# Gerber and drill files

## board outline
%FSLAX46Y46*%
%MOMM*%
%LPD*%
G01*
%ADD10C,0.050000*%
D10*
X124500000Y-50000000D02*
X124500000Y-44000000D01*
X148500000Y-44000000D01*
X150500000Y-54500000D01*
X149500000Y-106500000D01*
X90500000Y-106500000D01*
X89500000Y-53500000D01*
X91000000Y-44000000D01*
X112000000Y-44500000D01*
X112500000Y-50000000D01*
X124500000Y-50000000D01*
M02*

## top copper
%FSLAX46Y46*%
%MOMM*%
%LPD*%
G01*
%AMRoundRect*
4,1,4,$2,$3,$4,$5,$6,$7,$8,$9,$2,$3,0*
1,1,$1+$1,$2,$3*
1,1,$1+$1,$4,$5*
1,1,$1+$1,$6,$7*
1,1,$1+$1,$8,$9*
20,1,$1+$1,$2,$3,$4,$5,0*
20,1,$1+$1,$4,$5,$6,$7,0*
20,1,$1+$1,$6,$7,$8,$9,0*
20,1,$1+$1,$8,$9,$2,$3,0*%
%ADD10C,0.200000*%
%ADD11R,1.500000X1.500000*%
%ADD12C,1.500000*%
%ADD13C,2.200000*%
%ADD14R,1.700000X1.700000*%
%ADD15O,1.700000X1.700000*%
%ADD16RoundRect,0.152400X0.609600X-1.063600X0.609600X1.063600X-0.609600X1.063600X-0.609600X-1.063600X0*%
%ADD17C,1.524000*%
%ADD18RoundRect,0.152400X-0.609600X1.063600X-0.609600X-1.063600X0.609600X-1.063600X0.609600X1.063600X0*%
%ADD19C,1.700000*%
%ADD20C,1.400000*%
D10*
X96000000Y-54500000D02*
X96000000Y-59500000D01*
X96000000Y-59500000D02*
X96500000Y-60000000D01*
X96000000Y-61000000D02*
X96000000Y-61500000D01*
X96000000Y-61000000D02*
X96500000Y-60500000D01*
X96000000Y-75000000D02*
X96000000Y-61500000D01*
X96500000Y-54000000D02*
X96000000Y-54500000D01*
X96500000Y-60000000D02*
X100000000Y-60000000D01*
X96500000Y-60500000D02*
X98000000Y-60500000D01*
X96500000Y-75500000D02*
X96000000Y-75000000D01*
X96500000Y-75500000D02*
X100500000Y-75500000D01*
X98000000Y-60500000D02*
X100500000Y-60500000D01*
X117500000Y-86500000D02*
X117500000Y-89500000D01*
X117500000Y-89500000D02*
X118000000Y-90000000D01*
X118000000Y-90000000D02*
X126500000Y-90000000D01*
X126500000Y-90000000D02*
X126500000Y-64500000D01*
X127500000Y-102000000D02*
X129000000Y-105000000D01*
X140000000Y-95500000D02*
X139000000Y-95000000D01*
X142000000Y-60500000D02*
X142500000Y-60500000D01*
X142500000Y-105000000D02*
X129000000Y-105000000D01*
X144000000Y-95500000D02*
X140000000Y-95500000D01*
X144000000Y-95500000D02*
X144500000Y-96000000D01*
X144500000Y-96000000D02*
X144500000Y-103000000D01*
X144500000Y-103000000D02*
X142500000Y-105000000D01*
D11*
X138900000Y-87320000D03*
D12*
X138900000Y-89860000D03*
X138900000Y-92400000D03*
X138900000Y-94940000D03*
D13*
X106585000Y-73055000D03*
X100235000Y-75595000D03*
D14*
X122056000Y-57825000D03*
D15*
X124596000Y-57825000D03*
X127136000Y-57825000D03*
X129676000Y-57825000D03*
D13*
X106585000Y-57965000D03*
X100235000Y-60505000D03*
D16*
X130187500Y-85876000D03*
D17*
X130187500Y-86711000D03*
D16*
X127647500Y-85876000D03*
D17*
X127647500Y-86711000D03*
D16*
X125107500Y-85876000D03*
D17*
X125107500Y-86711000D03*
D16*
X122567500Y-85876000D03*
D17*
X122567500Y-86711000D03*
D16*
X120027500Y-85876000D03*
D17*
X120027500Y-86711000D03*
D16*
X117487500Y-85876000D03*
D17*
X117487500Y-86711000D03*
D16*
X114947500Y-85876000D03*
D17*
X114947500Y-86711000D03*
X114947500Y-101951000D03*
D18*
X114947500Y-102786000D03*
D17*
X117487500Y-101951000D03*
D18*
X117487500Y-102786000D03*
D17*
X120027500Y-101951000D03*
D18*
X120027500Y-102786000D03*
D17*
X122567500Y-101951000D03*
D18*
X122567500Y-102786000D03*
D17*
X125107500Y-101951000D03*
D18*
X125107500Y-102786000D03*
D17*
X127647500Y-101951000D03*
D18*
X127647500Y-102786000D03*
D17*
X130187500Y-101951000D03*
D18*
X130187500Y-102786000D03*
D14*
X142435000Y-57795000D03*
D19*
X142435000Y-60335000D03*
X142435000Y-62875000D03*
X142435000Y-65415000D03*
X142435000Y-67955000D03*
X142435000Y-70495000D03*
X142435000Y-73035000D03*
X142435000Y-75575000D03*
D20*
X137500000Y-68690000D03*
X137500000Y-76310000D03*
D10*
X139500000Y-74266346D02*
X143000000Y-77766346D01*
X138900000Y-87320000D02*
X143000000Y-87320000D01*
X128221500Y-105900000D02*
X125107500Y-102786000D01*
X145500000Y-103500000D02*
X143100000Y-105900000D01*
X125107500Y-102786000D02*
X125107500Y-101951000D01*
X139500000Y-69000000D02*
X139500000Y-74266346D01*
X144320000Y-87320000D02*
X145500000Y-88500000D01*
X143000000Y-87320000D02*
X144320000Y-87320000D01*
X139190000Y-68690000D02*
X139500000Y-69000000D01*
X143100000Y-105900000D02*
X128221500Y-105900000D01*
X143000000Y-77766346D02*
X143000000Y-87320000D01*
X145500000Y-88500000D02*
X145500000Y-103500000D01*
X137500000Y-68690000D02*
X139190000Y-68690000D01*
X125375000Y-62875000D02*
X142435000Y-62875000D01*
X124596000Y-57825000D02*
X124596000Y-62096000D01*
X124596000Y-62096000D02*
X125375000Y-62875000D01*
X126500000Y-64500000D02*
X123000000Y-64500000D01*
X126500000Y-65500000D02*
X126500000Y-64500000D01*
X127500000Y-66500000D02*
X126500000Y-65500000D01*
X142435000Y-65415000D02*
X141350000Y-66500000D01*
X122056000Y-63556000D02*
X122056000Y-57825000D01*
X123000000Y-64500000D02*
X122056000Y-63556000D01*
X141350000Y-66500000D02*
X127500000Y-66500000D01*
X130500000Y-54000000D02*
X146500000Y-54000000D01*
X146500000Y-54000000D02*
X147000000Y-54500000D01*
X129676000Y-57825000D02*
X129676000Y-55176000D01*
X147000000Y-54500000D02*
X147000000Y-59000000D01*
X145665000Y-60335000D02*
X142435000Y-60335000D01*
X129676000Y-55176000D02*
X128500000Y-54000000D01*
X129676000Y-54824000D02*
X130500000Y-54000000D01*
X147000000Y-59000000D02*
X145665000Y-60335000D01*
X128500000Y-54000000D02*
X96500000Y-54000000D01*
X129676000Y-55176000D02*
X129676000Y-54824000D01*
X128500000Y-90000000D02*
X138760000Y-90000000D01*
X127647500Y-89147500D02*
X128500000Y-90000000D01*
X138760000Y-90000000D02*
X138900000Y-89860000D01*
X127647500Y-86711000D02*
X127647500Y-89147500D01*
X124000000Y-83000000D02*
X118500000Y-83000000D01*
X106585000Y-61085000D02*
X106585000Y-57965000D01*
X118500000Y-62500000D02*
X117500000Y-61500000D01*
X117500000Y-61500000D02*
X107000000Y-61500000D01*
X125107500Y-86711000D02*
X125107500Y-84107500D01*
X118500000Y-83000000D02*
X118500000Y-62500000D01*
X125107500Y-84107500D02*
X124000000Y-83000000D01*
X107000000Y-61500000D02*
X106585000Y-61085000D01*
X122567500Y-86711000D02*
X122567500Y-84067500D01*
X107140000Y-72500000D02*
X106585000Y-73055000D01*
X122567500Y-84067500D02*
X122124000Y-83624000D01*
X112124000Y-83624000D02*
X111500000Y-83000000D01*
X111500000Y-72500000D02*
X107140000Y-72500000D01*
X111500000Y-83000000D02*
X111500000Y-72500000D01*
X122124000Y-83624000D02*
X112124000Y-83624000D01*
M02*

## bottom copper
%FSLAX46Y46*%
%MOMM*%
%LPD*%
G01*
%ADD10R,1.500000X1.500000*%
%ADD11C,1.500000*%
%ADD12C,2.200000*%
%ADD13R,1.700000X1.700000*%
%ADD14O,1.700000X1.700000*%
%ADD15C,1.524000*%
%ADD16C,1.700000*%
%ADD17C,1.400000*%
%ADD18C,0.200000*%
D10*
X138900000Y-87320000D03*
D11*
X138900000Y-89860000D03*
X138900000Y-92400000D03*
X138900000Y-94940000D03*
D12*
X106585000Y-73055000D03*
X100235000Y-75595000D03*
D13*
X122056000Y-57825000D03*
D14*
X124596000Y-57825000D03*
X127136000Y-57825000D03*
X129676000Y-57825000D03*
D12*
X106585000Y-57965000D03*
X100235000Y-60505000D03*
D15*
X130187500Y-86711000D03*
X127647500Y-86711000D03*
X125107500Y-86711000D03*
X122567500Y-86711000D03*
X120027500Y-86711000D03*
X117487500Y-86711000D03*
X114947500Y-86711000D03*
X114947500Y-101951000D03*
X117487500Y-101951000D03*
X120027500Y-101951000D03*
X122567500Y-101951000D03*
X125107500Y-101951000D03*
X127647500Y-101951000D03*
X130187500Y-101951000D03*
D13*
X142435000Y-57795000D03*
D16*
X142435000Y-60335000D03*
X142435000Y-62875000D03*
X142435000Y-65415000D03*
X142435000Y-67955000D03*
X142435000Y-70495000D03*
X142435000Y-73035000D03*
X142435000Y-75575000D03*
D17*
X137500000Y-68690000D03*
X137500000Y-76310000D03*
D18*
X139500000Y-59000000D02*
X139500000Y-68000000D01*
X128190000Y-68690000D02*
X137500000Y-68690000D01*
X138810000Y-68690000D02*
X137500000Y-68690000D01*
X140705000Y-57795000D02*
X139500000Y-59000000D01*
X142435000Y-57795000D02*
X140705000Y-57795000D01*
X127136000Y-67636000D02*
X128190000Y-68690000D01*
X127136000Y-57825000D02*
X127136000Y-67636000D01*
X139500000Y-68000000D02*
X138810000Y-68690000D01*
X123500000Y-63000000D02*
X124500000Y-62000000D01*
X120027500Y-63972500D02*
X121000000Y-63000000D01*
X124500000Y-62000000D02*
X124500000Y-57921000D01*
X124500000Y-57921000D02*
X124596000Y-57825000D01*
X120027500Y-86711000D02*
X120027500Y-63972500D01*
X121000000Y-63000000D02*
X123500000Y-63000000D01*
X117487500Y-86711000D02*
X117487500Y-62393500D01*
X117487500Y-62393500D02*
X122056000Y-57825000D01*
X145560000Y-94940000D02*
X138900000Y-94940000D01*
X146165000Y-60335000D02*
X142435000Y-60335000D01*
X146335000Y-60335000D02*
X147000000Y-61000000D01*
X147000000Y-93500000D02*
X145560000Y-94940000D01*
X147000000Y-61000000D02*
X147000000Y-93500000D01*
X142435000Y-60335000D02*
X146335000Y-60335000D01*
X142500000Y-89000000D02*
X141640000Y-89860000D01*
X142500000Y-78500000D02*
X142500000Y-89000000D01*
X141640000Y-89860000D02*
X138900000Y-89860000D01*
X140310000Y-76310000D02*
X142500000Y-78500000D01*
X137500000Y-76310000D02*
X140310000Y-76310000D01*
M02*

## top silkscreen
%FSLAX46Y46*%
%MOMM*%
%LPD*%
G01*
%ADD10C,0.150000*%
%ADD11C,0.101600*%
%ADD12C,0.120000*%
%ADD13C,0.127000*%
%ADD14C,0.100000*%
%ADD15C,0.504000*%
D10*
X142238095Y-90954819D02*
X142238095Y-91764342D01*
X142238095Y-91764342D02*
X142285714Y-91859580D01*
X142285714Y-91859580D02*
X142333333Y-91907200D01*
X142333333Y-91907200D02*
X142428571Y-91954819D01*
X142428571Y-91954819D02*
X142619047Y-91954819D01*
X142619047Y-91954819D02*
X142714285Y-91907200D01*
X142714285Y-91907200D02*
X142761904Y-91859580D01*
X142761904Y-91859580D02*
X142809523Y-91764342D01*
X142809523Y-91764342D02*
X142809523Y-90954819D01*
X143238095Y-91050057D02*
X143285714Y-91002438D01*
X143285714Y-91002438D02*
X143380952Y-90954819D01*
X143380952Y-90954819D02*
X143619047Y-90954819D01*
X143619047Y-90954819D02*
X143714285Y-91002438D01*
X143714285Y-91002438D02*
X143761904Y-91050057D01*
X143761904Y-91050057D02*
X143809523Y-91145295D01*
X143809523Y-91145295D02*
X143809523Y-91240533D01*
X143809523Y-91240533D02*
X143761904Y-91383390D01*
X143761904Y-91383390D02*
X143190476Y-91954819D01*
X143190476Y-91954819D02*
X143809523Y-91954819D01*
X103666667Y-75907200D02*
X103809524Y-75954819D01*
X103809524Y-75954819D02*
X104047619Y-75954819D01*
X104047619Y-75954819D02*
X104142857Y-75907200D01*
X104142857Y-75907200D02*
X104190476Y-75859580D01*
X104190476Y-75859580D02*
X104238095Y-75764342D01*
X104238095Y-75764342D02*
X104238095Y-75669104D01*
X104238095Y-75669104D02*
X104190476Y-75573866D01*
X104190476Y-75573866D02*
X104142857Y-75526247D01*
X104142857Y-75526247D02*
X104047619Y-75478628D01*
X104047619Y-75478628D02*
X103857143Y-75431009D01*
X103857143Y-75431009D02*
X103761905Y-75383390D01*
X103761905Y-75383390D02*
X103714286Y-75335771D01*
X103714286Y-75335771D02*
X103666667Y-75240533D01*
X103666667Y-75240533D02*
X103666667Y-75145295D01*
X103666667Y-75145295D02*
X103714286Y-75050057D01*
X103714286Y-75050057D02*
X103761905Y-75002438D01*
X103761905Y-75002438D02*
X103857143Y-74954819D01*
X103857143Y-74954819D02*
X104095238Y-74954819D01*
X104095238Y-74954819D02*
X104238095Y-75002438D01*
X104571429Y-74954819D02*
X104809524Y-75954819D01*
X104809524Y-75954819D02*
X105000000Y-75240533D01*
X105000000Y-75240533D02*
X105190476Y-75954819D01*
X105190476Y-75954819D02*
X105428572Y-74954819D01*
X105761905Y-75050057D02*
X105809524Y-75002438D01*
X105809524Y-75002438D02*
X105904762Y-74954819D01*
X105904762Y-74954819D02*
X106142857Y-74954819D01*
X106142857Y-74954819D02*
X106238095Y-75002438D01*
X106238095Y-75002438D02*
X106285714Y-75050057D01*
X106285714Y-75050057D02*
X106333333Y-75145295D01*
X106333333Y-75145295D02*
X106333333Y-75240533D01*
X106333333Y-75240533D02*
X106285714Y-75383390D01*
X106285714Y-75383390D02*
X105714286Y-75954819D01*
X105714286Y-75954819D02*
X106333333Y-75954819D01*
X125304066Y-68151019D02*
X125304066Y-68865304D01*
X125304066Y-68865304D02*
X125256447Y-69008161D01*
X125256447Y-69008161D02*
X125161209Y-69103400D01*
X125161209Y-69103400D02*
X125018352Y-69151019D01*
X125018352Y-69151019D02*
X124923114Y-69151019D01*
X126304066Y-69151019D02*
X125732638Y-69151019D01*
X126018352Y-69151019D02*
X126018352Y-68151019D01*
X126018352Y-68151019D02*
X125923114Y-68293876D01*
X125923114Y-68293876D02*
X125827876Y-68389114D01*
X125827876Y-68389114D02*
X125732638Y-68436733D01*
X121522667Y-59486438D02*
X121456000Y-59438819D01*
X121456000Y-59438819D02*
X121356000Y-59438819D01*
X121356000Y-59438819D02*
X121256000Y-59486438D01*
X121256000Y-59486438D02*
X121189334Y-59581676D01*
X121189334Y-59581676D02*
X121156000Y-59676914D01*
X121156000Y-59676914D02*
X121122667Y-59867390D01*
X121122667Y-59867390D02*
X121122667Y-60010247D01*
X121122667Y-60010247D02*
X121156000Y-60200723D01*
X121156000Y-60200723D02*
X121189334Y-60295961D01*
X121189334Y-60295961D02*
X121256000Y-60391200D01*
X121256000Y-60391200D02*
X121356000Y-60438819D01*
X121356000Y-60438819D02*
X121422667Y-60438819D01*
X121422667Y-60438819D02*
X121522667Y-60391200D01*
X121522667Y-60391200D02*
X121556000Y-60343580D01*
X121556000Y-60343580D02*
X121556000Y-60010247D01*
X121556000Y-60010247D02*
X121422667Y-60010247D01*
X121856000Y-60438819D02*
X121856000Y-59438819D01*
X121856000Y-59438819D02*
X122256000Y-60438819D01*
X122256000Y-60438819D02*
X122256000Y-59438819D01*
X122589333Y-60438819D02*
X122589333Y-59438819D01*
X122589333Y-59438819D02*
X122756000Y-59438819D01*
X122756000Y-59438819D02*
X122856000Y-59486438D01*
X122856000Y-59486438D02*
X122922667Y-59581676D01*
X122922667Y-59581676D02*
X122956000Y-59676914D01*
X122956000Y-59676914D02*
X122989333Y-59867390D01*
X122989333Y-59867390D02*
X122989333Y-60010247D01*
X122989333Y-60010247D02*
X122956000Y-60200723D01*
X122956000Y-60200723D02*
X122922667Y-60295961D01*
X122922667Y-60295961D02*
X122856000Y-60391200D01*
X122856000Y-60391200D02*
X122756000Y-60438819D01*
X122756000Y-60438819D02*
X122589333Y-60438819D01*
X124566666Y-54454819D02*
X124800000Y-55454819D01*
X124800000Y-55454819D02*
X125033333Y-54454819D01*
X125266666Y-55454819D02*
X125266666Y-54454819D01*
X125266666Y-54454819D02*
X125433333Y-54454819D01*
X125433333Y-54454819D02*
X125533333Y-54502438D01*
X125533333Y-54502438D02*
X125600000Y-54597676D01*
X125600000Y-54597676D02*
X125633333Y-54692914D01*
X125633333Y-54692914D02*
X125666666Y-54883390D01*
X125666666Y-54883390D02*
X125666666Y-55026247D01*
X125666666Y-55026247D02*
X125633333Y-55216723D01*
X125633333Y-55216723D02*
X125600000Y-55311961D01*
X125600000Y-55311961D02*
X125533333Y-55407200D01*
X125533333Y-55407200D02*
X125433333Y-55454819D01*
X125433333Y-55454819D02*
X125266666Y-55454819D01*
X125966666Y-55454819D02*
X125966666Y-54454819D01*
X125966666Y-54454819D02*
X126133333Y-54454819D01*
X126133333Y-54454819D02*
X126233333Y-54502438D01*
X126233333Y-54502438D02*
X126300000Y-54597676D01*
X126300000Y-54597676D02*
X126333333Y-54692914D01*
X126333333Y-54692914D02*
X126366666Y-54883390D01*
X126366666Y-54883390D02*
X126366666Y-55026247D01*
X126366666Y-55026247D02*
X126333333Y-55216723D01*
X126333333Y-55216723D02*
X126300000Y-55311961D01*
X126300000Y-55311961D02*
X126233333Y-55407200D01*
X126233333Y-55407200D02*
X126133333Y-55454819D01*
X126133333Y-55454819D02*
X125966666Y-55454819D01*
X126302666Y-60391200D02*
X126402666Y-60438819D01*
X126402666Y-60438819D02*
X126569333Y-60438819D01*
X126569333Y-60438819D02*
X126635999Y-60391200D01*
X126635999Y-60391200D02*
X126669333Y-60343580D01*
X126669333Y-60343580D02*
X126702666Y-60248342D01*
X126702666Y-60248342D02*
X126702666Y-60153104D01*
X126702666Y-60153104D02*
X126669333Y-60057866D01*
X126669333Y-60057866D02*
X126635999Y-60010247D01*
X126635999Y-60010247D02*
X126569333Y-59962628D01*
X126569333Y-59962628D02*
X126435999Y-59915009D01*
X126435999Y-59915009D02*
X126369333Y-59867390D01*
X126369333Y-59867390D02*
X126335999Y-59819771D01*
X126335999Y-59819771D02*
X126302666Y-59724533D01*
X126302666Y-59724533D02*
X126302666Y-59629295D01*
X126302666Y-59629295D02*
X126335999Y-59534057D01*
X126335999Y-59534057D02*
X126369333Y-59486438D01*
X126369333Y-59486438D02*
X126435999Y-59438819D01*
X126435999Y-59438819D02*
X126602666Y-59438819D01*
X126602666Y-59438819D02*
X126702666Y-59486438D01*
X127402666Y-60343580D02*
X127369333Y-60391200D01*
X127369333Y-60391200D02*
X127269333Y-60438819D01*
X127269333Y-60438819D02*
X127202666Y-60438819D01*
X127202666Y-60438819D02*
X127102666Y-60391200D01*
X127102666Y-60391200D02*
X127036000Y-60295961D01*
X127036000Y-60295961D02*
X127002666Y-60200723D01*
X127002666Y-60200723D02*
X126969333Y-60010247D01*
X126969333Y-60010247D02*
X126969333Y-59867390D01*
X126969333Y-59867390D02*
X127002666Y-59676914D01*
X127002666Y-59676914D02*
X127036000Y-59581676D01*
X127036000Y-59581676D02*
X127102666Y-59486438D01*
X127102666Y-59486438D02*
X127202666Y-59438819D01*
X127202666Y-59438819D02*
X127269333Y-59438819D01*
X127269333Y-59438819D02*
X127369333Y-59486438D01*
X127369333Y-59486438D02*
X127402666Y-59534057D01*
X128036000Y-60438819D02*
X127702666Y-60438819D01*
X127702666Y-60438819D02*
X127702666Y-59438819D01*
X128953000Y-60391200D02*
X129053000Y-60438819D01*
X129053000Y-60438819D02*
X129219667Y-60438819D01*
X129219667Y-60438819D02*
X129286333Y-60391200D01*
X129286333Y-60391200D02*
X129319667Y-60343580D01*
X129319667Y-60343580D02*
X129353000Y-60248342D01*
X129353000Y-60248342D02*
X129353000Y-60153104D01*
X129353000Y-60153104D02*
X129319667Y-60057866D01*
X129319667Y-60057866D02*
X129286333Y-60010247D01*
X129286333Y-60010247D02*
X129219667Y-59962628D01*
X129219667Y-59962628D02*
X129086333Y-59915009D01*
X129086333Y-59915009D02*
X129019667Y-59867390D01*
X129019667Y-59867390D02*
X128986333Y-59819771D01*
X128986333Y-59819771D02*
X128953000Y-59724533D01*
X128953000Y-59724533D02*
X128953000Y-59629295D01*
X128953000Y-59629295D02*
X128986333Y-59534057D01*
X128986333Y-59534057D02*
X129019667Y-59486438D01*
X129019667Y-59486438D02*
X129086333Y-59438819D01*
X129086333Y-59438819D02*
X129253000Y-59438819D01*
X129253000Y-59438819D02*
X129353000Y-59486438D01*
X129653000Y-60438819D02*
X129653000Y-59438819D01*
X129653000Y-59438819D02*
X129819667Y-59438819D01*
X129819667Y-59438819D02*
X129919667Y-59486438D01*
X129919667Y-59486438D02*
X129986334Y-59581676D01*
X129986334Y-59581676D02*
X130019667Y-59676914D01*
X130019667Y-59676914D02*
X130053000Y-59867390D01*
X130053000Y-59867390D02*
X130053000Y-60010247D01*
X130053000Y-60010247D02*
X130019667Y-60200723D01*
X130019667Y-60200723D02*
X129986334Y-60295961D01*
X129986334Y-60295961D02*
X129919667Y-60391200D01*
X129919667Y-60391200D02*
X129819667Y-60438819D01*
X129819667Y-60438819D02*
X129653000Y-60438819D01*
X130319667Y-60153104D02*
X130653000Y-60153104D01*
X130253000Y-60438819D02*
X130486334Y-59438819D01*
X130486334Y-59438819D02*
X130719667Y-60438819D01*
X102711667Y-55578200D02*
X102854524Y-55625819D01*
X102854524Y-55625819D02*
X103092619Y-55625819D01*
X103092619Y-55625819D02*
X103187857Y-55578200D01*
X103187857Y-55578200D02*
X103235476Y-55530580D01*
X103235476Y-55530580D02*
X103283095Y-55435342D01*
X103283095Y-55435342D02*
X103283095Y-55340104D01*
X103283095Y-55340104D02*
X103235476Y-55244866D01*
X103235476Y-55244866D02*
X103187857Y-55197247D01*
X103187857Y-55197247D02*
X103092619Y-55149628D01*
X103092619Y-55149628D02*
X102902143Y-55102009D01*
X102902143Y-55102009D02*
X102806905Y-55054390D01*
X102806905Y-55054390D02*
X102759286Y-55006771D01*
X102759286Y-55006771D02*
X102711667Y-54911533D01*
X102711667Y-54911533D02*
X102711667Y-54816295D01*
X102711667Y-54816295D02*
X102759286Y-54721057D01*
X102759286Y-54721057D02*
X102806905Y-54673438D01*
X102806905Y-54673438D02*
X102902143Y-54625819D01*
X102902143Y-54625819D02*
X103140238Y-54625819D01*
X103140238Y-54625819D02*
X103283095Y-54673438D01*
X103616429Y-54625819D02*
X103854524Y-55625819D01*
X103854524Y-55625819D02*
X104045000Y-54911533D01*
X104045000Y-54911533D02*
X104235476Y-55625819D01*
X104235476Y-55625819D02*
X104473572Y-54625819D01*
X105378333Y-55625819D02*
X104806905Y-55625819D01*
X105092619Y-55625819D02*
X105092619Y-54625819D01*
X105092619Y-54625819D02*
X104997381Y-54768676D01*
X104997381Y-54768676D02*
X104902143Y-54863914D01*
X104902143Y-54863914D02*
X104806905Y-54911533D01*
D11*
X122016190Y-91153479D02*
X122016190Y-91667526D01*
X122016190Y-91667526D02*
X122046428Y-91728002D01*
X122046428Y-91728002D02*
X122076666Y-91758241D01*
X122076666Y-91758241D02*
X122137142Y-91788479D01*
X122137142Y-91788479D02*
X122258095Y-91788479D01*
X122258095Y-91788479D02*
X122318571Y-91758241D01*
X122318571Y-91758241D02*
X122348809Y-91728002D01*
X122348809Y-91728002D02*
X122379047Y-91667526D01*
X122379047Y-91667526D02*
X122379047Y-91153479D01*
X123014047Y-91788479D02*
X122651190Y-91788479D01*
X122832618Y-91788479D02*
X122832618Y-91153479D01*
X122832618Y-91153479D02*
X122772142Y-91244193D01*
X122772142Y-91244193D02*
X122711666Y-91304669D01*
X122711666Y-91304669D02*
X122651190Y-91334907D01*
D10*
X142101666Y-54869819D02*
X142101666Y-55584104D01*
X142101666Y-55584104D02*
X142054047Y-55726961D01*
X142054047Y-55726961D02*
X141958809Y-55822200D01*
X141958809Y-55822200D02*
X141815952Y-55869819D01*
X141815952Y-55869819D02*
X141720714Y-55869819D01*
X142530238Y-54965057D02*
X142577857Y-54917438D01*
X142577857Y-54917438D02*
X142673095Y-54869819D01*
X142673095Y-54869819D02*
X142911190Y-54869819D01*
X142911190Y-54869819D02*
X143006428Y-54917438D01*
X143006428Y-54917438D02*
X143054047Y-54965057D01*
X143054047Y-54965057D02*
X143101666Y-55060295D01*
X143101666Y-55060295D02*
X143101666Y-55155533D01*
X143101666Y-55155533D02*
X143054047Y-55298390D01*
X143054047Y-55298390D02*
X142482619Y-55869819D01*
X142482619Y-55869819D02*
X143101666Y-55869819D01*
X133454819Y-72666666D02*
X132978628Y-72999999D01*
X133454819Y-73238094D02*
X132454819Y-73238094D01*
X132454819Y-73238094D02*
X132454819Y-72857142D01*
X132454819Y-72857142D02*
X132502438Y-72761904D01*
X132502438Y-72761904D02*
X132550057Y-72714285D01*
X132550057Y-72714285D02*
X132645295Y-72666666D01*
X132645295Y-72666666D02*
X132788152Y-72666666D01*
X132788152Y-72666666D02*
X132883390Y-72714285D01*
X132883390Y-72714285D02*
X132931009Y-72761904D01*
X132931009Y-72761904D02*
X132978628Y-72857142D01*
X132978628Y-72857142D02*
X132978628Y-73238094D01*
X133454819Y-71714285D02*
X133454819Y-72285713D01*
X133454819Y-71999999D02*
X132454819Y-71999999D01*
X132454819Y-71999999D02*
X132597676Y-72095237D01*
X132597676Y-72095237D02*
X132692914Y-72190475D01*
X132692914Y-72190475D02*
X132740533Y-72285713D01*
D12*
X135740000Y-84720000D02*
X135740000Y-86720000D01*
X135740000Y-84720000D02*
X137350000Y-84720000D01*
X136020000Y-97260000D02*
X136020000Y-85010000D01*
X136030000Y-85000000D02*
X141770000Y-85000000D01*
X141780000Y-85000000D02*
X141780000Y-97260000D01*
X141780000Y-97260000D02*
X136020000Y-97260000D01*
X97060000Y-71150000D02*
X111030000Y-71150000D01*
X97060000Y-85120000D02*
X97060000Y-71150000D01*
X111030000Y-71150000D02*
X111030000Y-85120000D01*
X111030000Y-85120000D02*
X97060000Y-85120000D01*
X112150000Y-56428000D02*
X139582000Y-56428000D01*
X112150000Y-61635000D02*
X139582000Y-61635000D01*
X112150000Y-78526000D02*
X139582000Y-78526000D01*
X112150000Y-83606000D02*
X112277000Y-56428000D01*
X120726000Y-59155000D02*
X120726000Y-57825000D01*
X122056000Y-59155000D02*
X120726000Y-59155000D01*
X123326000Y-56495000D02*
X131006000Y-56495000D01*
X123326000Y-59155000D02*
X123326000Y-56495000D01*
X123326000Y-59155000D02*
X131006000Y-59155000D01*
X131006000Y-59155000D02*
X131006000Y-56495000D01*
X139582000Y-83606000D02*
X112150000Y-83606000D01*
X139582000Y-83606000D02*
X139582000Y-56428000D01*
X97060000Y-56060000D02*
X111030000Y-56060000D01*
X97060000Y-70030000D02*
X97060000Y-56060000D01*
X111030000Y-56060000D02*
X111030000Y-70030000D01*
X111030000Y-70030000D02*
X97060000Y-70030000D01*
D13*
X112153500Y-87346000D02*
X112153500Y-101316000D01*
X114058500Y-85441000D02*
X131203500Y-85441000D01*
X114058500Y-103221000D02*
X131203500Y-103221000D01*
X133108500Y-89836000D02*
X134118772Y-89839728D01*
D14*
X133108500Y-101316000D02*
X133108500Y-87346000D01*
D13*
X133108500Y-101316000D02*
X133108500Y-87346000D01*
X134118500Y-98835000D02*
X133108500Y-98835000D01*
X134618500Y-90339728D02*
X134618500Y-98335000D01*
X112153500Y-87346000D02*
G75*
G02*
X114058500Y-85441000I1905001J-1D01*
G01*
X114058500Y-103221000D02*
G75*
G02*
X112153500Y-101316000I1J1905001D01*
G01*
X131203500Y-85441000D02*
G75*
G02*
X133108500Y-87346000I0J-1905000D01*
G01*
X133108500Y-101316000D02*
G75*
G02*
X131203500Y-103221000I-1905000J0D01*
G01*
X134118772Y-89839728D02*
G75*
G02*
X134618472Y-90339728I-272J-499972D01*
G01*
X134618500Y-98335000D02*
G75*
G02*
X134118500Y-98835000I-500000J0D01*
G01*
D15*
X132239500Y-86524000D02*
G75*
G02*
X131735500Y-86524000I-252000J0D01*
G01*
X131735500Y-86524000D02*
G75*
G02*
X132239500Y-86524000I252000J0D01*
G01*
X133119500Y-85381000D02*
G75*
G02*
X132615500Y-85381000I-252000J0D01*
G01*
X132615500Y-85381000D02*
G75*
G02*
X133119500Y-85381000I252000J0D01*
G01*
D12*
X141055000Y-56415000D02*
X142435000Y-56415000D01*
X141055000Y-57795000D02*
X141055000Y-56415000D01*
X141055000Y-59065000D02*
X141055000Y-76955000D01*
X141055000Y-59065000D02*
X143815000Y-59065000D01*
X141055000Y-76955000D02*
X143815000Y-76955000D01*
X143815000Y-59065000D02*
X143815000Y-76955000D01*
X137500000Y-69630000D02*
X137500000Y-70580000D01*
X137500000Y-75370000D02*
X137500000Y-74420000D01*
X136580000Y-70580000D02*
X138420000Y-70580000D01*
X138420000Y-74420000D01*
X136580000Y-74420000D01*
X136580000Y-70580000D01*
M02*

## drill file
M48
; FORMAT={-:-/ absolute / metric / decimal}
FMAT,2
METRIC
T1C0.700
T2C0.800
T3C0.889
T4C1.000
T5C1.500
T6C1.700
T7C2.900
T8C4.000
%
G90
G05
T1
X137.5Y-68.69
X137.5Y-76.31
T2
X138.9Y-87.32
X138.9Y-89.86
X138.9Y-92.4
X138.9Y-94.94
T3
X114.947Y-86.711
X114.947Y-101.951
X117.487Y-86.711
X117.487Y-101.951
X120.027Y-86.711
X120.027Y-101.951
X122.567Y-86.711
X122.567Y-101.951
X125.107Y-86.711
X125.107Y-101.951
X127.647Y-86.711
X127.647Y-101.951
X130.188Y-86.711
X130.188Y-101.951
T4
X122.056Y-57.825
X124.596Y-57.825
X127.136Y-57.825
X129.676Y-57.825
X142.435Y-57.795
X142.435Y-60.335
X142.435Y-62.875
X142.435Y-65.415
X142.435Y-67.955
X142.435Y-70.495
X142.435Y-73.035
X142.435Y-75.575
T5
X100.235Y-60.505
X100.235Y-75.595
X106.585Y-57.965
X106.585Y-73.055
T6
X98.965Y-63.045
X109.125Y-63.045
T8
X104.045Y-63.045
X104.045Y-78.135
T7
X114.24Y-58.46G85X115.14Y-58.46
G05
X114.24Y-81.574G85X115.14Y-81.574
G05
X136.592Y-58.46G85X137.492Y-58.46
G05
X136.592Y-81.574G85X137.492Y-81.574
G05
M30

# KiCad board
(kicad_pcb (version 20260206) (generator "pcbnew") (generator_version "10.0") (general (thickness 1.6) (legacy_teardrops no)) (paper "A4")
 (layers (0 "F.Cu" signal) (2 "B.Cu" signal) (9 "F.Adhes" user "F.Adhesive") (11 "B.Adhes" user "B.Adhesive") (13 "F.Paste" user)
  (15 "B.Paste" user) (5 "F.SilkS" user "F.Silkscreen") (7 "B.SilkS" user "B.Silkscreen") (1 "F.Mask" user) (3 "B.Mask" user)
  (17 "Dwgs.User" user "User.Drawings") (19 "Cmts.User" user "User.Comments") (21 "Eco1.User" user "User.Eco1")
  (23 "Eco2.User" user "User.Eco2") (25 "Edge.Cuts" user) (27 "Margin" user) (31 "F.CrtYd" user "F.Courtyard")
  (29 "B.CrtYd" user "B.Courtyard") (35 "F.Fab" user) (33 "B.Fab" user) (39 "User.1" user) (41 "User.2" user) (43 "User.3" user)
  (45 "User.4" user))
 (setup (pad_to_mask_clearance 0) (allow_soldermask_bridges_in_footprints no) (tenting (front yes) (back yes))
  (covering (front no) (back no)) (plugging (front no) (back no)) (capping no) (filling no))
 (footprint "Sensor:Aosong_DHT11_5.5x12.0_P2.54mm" (layer "F.Cu") (at 138.9 87.32)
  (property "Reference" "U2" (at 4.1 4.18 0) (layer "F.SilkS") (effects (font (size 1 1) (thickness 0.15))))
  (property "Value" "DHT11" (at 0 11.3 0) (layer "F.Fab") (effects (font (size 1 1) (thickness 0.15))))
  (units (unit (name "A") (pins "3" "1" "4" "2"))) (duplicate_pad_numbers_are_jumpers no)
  (fp_line (start -3.16 -2.6) (end -3.16 -0.6) (stroke (width 0.12) (type solid)) (layer "F.SilkS"))
  (fp_line (start -3.16 -2.6) (end -1.55 -2.6) (stroke (width 0.12) (type solid)) (layer "F.SilkS"))
  (fp_line (start -2.88 9.94) (end -2.88 -2.31) (stroke (width 0.12) (type solid)) (layer "F.SilkS"))
  (fp_line (start -2.87 -2.32) (end 2.87 -2.32) (stroke (width 0.12) (type solid)) (layer "F.SilkS"))
  (fp_line (start 2.88 -2.32) (end 2.88 9.94) (stroke (width 0.12) (type solid)) (layer "F.SilkS"))
  (fp_line (start 2.88 9.94) (end -2.88 9.94) (stroke (width 0.12) (type solid)) (layer "F.SilkS"))
  (pad "1" thru_hole rect (at 0 0) (size 1.5 1.5) (drill 0.8) (layers "*.Cu" "*.Mask") (remove_unused_layers no) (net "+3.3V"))
  (pad "2" thru_hole circle (at 0 2.54) (size 1.5 1.5) (drill 0.8) (layers "*.Cu" "*.Mask") (remove_unused_layers no) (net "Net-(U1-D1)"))
  (pad "3" thru_hole circle (at 0 5.08) (size 1.5 1.5) (drill 0.8) (layers "*.Cu" "*.Mask") (remove_unused_layers no)
   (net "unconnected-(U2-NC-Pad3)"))
  (pad "4" thru_hole circle (at 0 7.62) (size 1.5 1.5) (drill 0.8) (layers "*.Cu" "*.Mask") (remove_unused_layers no) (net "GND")))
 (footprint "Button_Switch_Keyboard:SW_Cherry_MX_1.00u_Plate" (layer "F.Cu") (at 106.585 73.055)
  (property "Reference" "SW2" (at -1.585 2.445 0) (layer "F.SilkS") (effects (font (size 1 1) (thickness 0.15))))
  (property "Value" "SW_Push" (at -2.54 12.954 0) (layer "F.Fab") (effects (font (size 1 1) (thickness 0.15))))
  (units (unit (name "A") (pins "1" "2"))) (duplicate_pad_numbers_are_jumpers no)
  (fp_line (start -9.525 -1.905) (end 4.445 -1.905) (stroke (width 0.12) (type solid)) (layer "F.SilkS"))
  (fp_line (start -9.525 12.065) (end -9.525 -1.905) (stroke (width 0.12) (type solid)) (layer "F.SilkS"))
  (fp_line (start 4.445 -1.905) (end 4.445 12.065) (stroke (width 0.12) (type solid)) (layer "F.SilkS"))
  (fp_line (start 4.445 12.065) (end -9.525 12.065) (stroke (width 0.12) (type solid)) (layer "F.SilkS"))
  (pad "" np_thru_hole circle (at -2.54 5.08) (size 4 4) (drill 4) (layers "*.Cu" "*.Mask"))
  (pad "1" thru_hole circle (at 0 0) (size 2.2 2.2) (drill 1.5) (layers "*.Cu" "*.Mask") (remove_unused_layers no) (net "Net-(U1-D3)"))
  (pad "2" thru_hole circle (at -6.35 2.54) (size 2.2 2.2) (drill 1.5) (layers "*.Cu" "*.Mask") (remove_unused_layers no) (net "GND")))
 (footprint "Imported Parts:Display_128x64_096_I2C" (layer "F.Cu") (at 125.866 57.825)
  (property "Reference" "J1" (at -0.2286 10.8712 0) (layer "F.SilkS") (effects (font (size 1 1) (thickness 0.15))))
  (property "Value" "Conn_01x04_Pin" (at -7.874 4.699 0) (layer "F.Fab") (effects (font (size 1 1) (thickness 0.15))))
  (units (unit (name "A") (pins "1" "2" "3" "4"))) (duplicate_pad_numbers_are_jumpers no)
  (fp_line (start -13.716 -1.397) (end 13.716 -1.397) (stroke (width 0.12) (type solid)) (layer "F.SilkS"))
  (fp_line (start -13.716 3.81) (end 13.716 3.81) (stroke (width 0.12) (type solid)) (layer "F.SilkS"))
  (fp_line (start -13.716 20.701) (end 13.716 20.701) (stroke (width 0.12) (type solid)) (layer "F.SilkS"))
  (fp_line (start -13.716 25.781) (end -13.589 -1.397) (stroke (width 0.12) (type solid)) (layer "F.SilkS"))
  (fp_line (start -5.14 1.33) (end -5.14 0) (stroke (width 0.12) (type solid)) (layer "F.SilkS"))
  (fp_line (start -3.81 1.33) (end -5.14 1.33) (stroke (width 0.12) (type solid)) (layer "F.SilkS"))
  (fp_line (start -2.54 -1.33) (end 5.14 -1.33) (stroke (width 0.12) (type solid)) (layer "F.SilkS"))
  (fp_line (start -2.54 1.33) (end -2.54 -1.33) (stroke (width 0.12) (type solid)) (layer "F.SilkS"))
  (fp_line (start -2.54 1.33) (end 5.14 1.33) (stroke (width 0.12) (type solid)) (layer "F.SilkS"))
  (fp_line (start 5.14 1.33) (end 5.14 -1.33) (stroke (width 0.12) (type solid)) (layer "F.SilkS"))
  (fp_line (start 13.716 25.781) (end -13.716 25.781) (stroke (width 0.12) (type solid)) (layer "F.SilkS"))
  (fp_line (start 13.716 25.781) (end 13.716 -1.397) (stroke (width 0.12) (type solid)) (layer "F.SilkS"))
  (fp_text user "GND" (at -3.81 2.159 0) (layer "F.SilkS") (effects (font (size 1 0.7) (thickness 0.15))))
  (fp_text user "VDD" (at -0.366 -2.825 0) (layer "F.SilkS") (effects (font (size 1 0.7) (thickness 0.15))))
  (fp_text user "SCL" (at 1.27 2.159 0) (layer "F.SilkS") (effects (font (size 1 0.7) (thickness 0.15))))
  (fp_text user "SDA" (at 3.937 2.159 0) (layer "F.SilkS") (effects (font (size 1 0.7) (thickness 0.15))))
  (pad "" np_thru_hole oval (at -11.176 0.635) (size 3.8 2.9) (drill oval 3.8 2.9) (layers "*.Cu" "*.Mask"))
  (pad "" np_thru_hole oval (at -11.176 23.749) (size 3.8 2.9) (drill oval 3.8 2.9) (layers "*.Cu" "*.Mask"))
  (pad "" np_thru_hole oval (at 11.176 0.635) (size 3.8 2.9) (drill oval 3.8 2.9) (layers "*.Cu" "*.Mask"))
  (pad "" np_thru_hole oval (at 11.176 23.749) (size 3.8 2.9) (drill oval 3.8 2.9) (layers "*.Cu" "*.Mask"))
  (pad "1" thru_hole rect (at -3.81 0 90) (size 1.7 1.7) (drill 1) (layers "*.Cu" "*.Mask") (remove_unused_layers no) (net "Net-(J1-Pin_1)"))
  (pad "2" thru_hole oval (at -1.27 0 90) (size 1.7 1.7) (drill 1) (layers "*.Cu" "*.Mask") (remove_unused_layers no) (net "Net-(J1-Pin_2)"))
  (pad "3" thru_hole oval (at 1.27 0 90) (size 1.7 1.7) (drill 1) (layers "*.Cu" "*.Mask") (remove_unused_layers no) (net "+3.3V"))
  (pad "4" thru_hole oval (at 3.81 0 90) (size 1.7 1.7) (drill 1) (layers "*.Cu" "*.Mask") (remove_unused_layers no) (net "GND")))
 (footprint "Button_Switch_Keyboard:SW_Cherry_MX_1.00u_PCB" (layer "F.Cu") (at 106.585 57.965)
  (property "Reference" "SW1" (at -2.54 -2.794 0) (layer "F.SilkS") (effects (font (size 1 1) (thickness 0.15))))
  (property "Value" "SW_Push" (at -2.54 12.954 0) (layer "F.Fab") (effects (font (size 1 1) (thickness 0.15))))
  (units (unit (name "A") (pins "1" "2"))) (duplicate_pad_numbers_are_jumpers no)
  (fp_line (start -9.525 -1.905) (end 4.445 -1.905) (stroke (width 0.12) (type solid)) (layer "F.SilkS"))
  (fp_line (start -9.525 12.065) (end -9.525 -1.905) (stroke (width 0.12) (type solid)) (layer "F.SilkS"))
  (fp_line (start 4.445 -1.905) (end 4.445 12.065) (stroke (width 0.12) (type solid)) (layer "F.SilkS"))
  (fp_line (start 4.445 12.065) (end -9.525 12.065) (stroke (width 0.12) (type solid)) (layer "F.SilkS"))
  (pad "" np_thru_hole circle (at -7.62 5.08) (size 1.7 1.7) (drill 1.7) (layers "*.Cu" "*.Mask"))
  (pad "" np_thru_hole circle (at -2.54 5.08) (size 4 4) (drill 4) (layers "*.Cu" "*.Mask"))
  (pad "" np_thru_hole circle (at 2.54 5.08) (size 1.7 1.7) (drill 1.7) (layers "*.Cu" "*.Mask"))
  (pad "1" thru_hole circle (at 0 0) (size 2.2 2.2) (drill 1.5) (layers "*.Cu" "*.Mask") (remove_unused_layers no) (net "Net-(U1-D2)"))
  (pad "2" thru_hole circle (at -6.35 2.54) (size 2.2 2.2) (drill 1.5) (layers "*.Cu" "*.Mask") (remove_unused_layers no) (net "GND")))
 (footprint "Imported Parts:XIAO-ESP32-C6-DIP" (layer "F.Cu") (at 122.5675 94.331)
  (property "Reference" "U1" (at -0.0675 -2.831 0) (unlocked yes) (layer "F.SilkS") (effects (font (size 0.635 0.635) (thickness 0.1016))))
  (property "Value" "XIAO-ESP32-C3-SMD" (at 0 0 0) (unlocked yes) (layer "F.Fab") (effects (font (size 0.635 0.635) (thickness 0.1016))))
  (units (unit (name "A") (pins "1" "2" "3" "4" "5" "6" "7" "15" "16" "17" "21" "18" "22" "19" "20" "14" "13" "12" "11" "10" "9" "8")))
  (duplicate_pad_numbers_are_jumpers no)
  (fp_line (start -10.414 -6.985) (end -10.414 6.985) (stroke (width 0.127) (type solid)) (layer "F.SilkS"))
  (fp_line (start -8.509 -8.89) (end 8.636 -8.89) (stroke (width 0.127) (type solid)) (layer "F.SilkS"))
  (fp_line (start -8.509 8.89) (end 8.636 8.89) (stroke (width 0.127) (type solid)) (layer "F.SilkS"))
  (fp_line (start 10.541 -4.495) (end 11.551272 -4.491272) (stroke (width 0.127) (type solid)) (layer "F.SilkS"))
  (fp_line (start 10.541 6.985) (end 10.541 -6.985) (stroke (width 0.1) (type solid)) (layer "F.SilkS"))
  (fp_line (start 10.541 6.985) (end 10.541 -6.985) (stroke (width 0.127) (type solid)) (layer "F.SilkS"))
  (fp_line (start 11.551 4.504) (end 10.541 4.504) (stroke (width 0.127) (type solid)) (layer "F.SilkS"))
  (fp_line (start 12.051 -3.991272) (end 12.051 4.004) (stroke (width 0.127) (type solid)) (layer "F.SilkS"))
  (fp_arc (start -10.414 -6.985) (mid -9.856038 -8.332038) (end -8.509 -8.89) (stroke (width 0.127) (type solid)) (layer "F.SilkS"))
  (fp_arc (start -8.509 8.89) (mid -9.856038 8.332038) (end -10.414 6.985) (stroke (width 0.127) (type solid)) (layer "F.SilkS"))
  (fp_arc (start 8.636 -8.89) (mid 9.983038 -8.332038) (end 10.541 -6.985) (stroke (width 0.127) (type solid)) (layer "F.SilkS"))
  (fp_arc (start 10.541 6.985) (mid 9.983038 8.332038) (end 8.636 8.89) (stroke (width 0.127) (type solid)) (layer "F.SilkS"))
  (fp_arc (start 11.551272 -4.491272) (mid 11.904644 -4.344724) (end 12.051 -3.991272) (stroke (width 0.127) (type default))
   (layer "F.SilkS"))
  (fp_arc (start 12.051 4.004) (mid 11.904553 4.357553) (end 11.551 4.504) (stroke (width 0.127) (type default)) (layer "F.SilkS"))
  (fp_circle (center 9.42 -7.807) (end 9.674 -7.807) (stroke (width 0.5) (type solid)) (fill yes) (layer "F.SilkS"))
  (fp_circle (center 10.3 -8.95) (end 10.554 -8.95) (stroke (width 0.5) (type solid)) (fill yes) (layer "F.SilkS"))
  (pad "1" smd roundrect (at 7.62 -8.455 90) (size 2.432 1.524) (layers "F.Cu" "F.Mask") (roundrect_rratio 0.1)
   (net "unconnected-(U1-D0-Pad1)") (thermal_bridge_angle 45))
  (pad "1" thru_hole circle (at 7.62 -7.62 90) (size 1.524 1.524) (drill 0.889) (layers "*.Cu" "*.Mask") (remove_unused_layers no)
   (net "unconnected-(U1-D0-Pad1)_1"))
  (pad "2" smd roundrect (at 5.08 -8.455 90) (size 2.432 1.524) (layers "F.Cu" "F.Mask") (roundrect_rratio 0.1) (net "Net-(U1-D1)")
   (thermal_bridge_angle 45))
  (pad "2" thru_hole circle (at 5.08 -7.62 90) (size 1.524 1.524) (drill 0.889) (layers "*.Cu" "*.Mask") (remove_unused_layers no)
   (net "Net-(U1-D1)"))
  (pad "3" smd roundrect (at 2.54 -8.455 90) (size 2.432 1.524) (layers "F.Cu" "F.Mask") (roundrect_rratio 0.1) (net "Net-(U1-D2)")
   (thermal_bridge_angle 45))
  (pad "3" thru_hole circle (at 2.54 -7.62 90) (size 1.524 1.524) (drill 0.889) (layers "*.Cu" "*.Mask") (remove_unused_layers no)
   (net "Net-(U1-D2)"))
  (pad "4" smd roundrect (at 0 -8.455 90) (size 2.432 1.524) (layers "F.Cu" "F.Mask") (roundrect_rratio 0.1) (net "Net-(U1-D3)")
   (thermal_bridge_angle 45))
  (pad "4" thru_hole circle (at 0 -7.62 90) (size 1.524 1.524) (drill 0.889) (layers "*.Cu" "*.Mask") (remove_unused_layers no)
   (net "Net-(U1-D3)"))
  (pad "5" smd roundrect (at -2.54 -8.455 90) (size 2.432 1.524) (layers "F.Cu" "F.Mask") (roundrect_rratio 0.1) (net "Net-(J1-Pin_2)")
   (thermal_bridge_angle 45))
  (pad "5" thru_hole circle (at -2.54 -7.62 90) (size 1.524 1.524) (drill 0.889) (layers "*.Cu" "*.Mask") (remove_unused_layers no)
   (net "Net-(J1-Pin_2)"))
  (pad "6" smd roundrect (at -5.08 -8.455 90) (size 2.432 1.524) (layers "F.Cu" "F.Mask") (roundrect_rratio 0.1) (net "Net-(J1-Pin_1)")
   (thermal_bridge_angle 45))
  (pad "6" thru_hole circle (at -5.08 -7.62 90) (size 1.524 1.524) (drill 0.889) (layers "*.Cu" "*.Mask") (remove_unused_layers no)
   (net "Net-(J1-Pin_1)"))
  (pad "7" smd roundrect (at -7.62 -8.455 90) (size 2.432 1.524) (layers "F.Cu" "F.Mask") (roundrect_rratio 0.1)
   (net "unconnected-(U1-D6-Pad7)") (thermal_bridge_angle 45))
  (pad "7" thru_hole circle (at -7.62 -7.62 90) (size 1.524 1.524) (drill 0.889) (layers "*.Cu" "*.Mask") (remove_unused_layers no)
   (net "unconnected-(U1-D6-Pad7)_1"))
  (pad "8" thru_hole circle (at -7.62 7.62 270) (size 1.524 1.524) (drill 0.889) (layers "*.Cu" "*.Mask") (remove_unused_layers no)
   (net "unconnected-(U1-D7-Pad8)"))
  (pad "8" smd roundrect (at -7.62 8.455 270) (size 2.432 1.524) (layers "F.Cu" "F.Mask") (roundrect_rratio 0.1)
   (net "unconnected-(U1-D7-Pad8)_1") (thermal_bridge_angle 45))
  (pad "9" thru_hole circle (at -5.08 7.62 270) (size 1.524 1.524) (drill 0.889) (layers "*.Cu" "*.Mask") (remove_unused_layers no)
   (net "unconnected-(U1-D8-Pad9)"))
  (pad "9" smd roundrect (at -5.08 8.455 270) (size 2.432 1.524) (layers "F.Cu" "F.Mask") (roundrect_rratio 0.1)
   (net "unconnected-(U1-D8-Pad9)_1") (thermal_bridge_angle 45))
  (pad "10" thru_hole circle (at -2.54 7.62 270) (size 1.524 1.524) (drill 0.889) (layers "*.Cu" "*.Mask") (remove_unused_layers no)
   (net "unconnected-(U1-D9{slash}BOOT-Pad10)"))
  (pad "10" smd roundrect (at -2.54 8.455 270) (size 2.432 1.524) (layers "F.Cu" "F.Mask") (roundrect_rratio 0.1)
   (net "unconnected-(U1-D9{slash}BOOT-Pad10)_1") (thermal_bridge_angle 45))
  (pad "11" thru_hole circle (at 0 7.62 270) (size 1.524 1.524) (drill 0.889) (layers "*.Cu" "*.Mask") (remove_unused_layers no)
   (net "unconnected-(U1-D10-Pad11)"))
  (pad "11" smd roundrect (at 0 8.455 270) (size 2.432 1.524) (layers "F.Cu" "F.Mask") (roundrect_rratio 0.1)
   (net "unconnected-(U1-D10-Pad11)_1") (thermal_bridge_angle 45))
  (pad "12" thru_hole circle (at 2.54 7.62 270) (size 1.524 1.524) (drill 0.889) (layers "*.Cu" "*.Mask") (remove_unused_layers no)
   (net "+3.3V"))
  (pad "12" smd roundrect (at 2.54 8.455 270) (size 2.432 1.524) (layers "F.Cu" "F.Mask") (roundrect_rratio 0.1) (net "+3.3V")
   (thermal_bridge_angle 45))
  (pad "13" thru_hole circle (at 5.08 7.62 270) (size 1.524 1.524) (drill 0.889) (layers "*.Cu" "*.Mask") (remove_unused_layers no)
   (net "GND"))
  (pad "13" smd roundrect (at 5.08 8.455 270) (size 2.432 1.524) (layers "F.Cu" "F.Mask") (roundrect_rratio 0.1) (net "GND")
   (thermal_bridge_angle 45))
  (pad "14" thru_hole circle (at 7.62 7.62 270) (size 1.524 1.524) (drill 0.889) (layers "*.Cu" "*.Mask") (remove_unused_layers no)
   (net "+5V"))
  (pad "14" smd roundrect (at 7.62 8.455 270) (size 2.432 1.524) (layers "F.Cu" "F.Mask") (roundrect_rratio 0.1) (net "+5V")
   (thermal_bridge_angle 45)))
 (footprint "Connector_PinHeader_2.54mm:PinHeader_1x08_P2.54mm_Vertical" (layer "F.Cu") (at 142.435 57.795)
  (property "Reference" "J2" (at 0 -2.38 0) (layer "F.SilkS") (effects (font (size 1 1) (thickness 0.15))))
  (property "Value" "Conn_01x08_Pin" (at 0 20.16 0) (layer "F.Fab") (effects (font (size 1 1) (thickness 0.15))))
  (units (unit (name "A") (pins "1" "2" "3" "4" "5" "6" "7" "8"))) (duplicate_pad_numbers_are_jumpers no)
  (fp_line (start -1.38 -1.38) (end 0 -1.38) (stroke (width 0.12) (type solid)) (layer "F.SilkS"))
  (fp_line (start -1.38 0) (end -1.38 -1.38) (stroke (width 0.12) (type solid)) (layer "F.SilkS"))
  (fp_line (start -1.38 1.27) (end -1.38 19.16) (stroke (width 0.12) (type solid)) (layer "F.SilkS"))
  (fp_line (start -1.38 1.27) (end 1.38 1.27) (stroke (width 0.12) (type solid)) (layer "F.SilkS"))
  (fp_line (start -1.38 19.16) (end 1.38 19.16) (stroke (width 0.12) (type solid)) (layer "F.SilkS"))
  (fp_line (start 1.38 1.27) (end 1.38 19.16) (stroke (width 0.12) (type solid)) (layer "F.SilkS"))
  (pad "1" thru_hole rect (at 0 0) (size 1.7 1.7) (drill 1) (layers "*.Cu" "*.Mask") (remove_unused_layers no) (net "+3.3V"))
  (pad "2" thru_hole circle (at 0 2.54) (size 1.7 1.7) (drill 1) (layers "*.Cu" "*.Mask") (remove_unused_layers no) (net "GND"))
  (pad "3" thru_hole circle (at 0 5.08) (size 1.7 1.7) (drill 1) (layers "*.Cu" "*.Mask") (remove_unused_layers no) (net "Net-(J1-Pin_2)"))
  (pad "4" thru_hole circle (at 0 7.62) (size 1.7 1.7) (drill 1) (layers "*.Cu" "*.Mask") (remove_unused_layers no) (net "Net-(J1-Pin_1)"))
  (pad "5" thru_hole circle (at 0 10.16) (size 1.7 1.7) (drill 1) (layers "*.Cu" "*.Mask") (remove_unused_layers no)
   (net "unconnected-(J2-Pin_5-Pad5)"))
  (pad "6" thru_hole circle (at 0 12.7) (size 1.7 1.7) (drill 1) (layers "*.Cu" "*.Mask") (remove_unused_layers no)
   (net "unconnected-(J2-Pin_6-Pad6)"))
  (pad "7" thru_hole circle (at 0 15.24) (size 1.7 1.7) (drill 1) (layers "*.Cu" "*.Mask") (remove_unused_layers no)
   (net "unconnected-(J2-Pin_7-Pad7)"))
  (pad "8" thru_hole circle (at 0 17.78) (size 1.7 1.7) (drill 1) (layers "*.Cu" "*.Mask") (remove_unused_layers no)
   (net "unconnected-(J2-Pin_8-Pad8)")))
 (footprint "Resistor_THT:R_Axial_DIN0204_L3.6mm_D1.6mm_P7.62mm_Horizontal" (layer "F.Cu") (at 137.5 68.69 -90)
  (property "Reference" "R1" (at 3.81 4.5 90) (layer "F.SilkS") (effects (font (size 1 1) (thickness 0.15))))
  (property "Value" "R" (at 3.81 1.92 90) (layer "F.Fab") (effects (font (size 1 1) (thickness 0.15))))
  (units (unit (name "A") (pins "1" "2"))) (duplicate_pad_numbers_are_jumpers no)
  (fp_line (start 0.94 0) (end 1.89 0) (stroke (width 0.12) (type solid)) (layer "F.SilkS"))
  (fp_line (start 6.68 0) (end 5.73 0) (stroke (width 0.12) (type solid)) (layer "F.SilkS"))
  (fp_rect (start 1.89 -0.92) (end 5.73 0.92) (stroke (width 0.12) (type solid)) (fill no) (layer "F.SilkS"))
  (pad "1" thru_hole circle (at 0 0 270) (size 1.4 1.4) (drill 0.7) (layers "*.Cu" "*.Mask") (remove_unused_layers no) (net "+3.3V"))
  (pad "2" thru_hole circle (at 7.62 0 270) (size 1.4 1.4) (drill 0.7) (layers "*.Cu" "*.Mask") (remove_unused_layers no)
   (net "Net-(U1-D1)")))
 (gr_line (start 96 54.5) (end 96 59.5) (stroke (width 0.2) (type default)) (layer "F.Cu") (net "GND"))
 (gr_line (start 96 59.5) (end 96.5 60) (stroke (width 0.2) (type default)) (layer "F.Cu") (net "GND"))
 (gr_line (start 96 61) (end 96 61.5) (stroke (width 0.2) (type default)) (layer "F.Cu") (net "GND"))
 (gr_line (start 96 61) (end 96.5 60.5) (stroke (width 0.2) (type default)) (layer "F.Cu") (net "GND"))
 (gr_line (start 96 75) (end 96 61.5) (stroke (width 0.2) (type default)) (layer "F.Cu") (net "GND"))
 (gr_line (start 96.5 54) (end 96 54.5) (stroke (width 0.2) (type default)) (layer "F.Cu") (net "GND"))
 (gr_line (start 96.5 60) (end 100 60) (stroke (width 0.2) (type default)) (layer "F.Cu") (net "GND"))
 (gr_line (start 96.5 60.5) (end 98 60.5) (stroke (width 0.2) (type default)) (layer "F.Cu") (net "GND"))
 (gr_line (start 96.5 75.5) (end 96 75) (stroke (width 0.2) (type default)) (layer "F.Cu") (net "GND"))
 (gr_line (start 96.5 75.5) (end 100.5 75.5) (stroke (width 0.2) (type default)) (layer "F.Cu") (net "GND"))
 (gr_line (start 98 60.5) (end 100.5 60.5) (stroke (width 0.2) (type default)) (layer "F.Cu") (net "GND"))
 (gr_line (start 117.5 86.5) (end 117.5 89.5) (stroke (width 0.2) (type default)) (layer "F.Cu") (net "Net-(J1-Pin_1)"))
 (gr_line (start 117.5 89.5) (end 118 90) (stroke (width 0.2) (type default)) (layer "F.Cu") (net "Net-(J1-Pin_1)"))
 (gr_line (start 118 90) (end 126.5 90) (stroke (width 0.2) (type default)) (layer "F.Cu") (net "Net-(J1-Pin_1)"))
 (gr_line (start 126.5 90) (end 126.5 64.5) (stroke (width 0.2) (type default)) (layer "F.Cu") (net "Net-(J1-Pin_1)"))
 (gr_line (start 127.5 102) (end 129 105) (stroke (width 0.2) (type default)) (layer "F.Cu") (net "GND"))
 (gr_line (start 140 95.5) (end 139 95) (stroke (width 0.2) (type default)) (layer "F.Cu") (net "GND"))
 (gr_line (start 142 60.5) (end 142.5 60.5) (stroke (width 0.2) (type default)) (layer "F.Cu") (net "GND"))
 (gr_line (start 142.5 105) (end 129 105) (stroke (width 0.2) (type default)) (layer "F.Cu") (net "GND"))
 (gr_line (start 144 95.5) (end 140 95.5) (stroke (width 0.2) (type default)) (layer "F.Cu") (net "GND"))
 (gr_line (start 144 95.5) (end 144.5 96) (stroke (width 0.2) (type default)) (layer "F.Cu") (net "GND"))
 (gr_line (start 144.5 96) (end 144.5 103) (stroke (width 0.2) (type default)) (layer "F.Cu") (net "GND"))
 (gr_line (start 144.5 103) (end 142.5 105) (stroke (width 0.2) (type default)) (layer "F.Cu") (net "GND"))
 (gr_poly
  (pts (xy 124.5 50) (xy 124.5 44) (xy 148.5 44) (xy 150.5 54.5) (xy 149.5 106.5) (xy 90.5 106.5) (xy 89.5 53.5) (xy 91 44) (xy 112 44.5)
   (xy 112.5 50))
  (stroke (width 0.05) (type solid)) (fill no) (layer "Edge.Cuts"))
 (segment (start 139.5 74.266346) (end 143 77.766346) (width 0.2) (layer "F.Cu") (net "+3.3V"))
 (segment (start 138.9 87.32) (end 143 87.32) (width 0.2) (layer "F.Cu") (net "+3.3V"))
 (segment (start 128.2215 105.9) (end 125.1075 102.786) (width 0.2) (layer "F.Cu") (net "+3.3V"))
 (segment (start 145.5 103.5) (end 143.1 105.9) (width 0.2) (layer "F.Cu") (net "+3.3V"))
 (segment (start 125.1075 102.786) (end 125.1075 101.951) (width 0.2) (layer "F.Cu") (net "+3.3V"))
 (segment (start 139.5 69) (end 139.5 74.266346) (width 0.2) (layer "F.Cu") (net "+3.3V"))
 (segment (start 144.32 87.32) (end 145.5 88.5) (width 0.2) (layer "F.Cu") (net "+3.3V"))
 (segment (start 143 87.32) (end 144.32 87.32) (width 0.2) (layer "F.Cu") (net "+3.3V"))
 (segment (start 139.19 68.69) (end 139.5 69) (width 0.2) (layer "F.Cu") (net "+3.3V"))
 (segment (start 143.1 105.9) (end 128.2215 105.9) (width 0.2) (layer "F.Cu") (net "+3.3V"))
 (segment (start 143 77.766346) (end 143 87.32) (width 0.2) (layer "F.Cu") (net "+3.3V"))
 (segment (start 145.5 88.5) (end 145.5 103.5) (width 0.2) (layer "F.Cu") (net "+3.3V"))
 (segment (start 137.5 68.69) (end 139.19 68.69) (width 0.2) (layer "F.Cu") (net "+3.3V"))
 (segment (start 139.5 59) (end 139.5 68) (width 0.2) (layer "B.Cu") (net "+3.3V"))
 (segment (start 128.19 68.69) (end 137.5 68.69) (width 0.2) (layer "B.Cu") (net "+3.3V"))
 (segment (start 138.81 68.69) (end 137.5 68.69) (width 0.2) (layer "B.Cu") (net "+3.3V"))
 (segment (start 140.705 57.795) (end 139.5 59) (width 0.2) (layer "B.Cu") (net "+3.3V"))
 (segment (start 142.435 57.795) (end 140.705 57.795) (width 0.2) (layer "B.Cu") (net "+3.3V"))
 (segment (start 127.136 67.636) (end 128.19 68.69) (width 0.2) (layer "B.Cu") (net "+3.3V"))
 (segment (start 127.136 57.825) (end 127.136 67.636) (width 0.2) (layer "B.Cu") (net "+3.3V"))
 (segment (start 139.5 68) (end 138.81 68.69) (width 0.2) (layer "B.Cu") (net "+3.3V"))
 (segment (start 125.375 62.875) (end 142.435 62.875) (width 0.2) (layer "F.Cu") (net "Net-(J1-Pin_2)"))
 (segment (start 124.596 57.825) (end 124.596 62.096) (width 0.2) (layer "F.Cu") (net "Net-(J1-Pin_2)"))
 (segment (start 124.596 62.096) (end 125.375 62.875) (width 0.2) (layer "F.Cu") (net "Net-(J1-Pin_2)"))
 (segment (start 123.5 63) (end 124.5 62) (width 0.2) (layer "B.Cu") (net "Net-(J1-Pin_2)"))
 (segment (start 120.0275 63.9725) (end 121 63) (width 0.2) (layer "B.Cu") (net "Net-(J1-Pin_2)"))
 (segment (start 124.5 62) (end 124.5 57.921) (width 0.2) (layer "B.Cu") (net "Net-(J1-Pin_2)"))
 (segment (start 124.5 57.921) (end 124.596 57.825) (width 0.2) (layer "B.Cu") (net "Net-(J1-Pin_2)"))
 (segment (start 120.0275 86.711) (end 120.0275 63.9725) (width 0.2) (layer "B.Cu") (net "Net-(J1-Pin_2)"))
 (segment (start 121 63) (end 123.5 63) (width 0.2) (layer "B.Cu") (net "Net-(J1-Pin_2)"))
 (segment (start 126.5 64.5) (end 123 64.5) (width 0.2) (layer "F.Cu") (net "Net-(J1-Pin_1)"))
 (segment (start 126.5 65.5) (end 126.5 64.5) (width 0.2) (layer "F.Cu") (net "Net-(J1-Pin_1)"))
 (segment (start 127.5 66.5) (end 126.5 65.5) (width 0.2) (layer "F.Cu") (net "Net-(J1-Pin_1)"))
 (segment (start 142.435 65.415) (end 141.35 66.5) (width 0.2) (layer "F.Cu") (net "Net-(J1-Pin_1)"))
 (segment (start 122.056 63.556) (end 122.056 57.825) (width 0.2) (layer "F.Cu") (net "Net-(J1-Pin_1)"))
 (segment (start 123 64.5) (end 122.056 63.556) (width 0.2) (layer "F.Cu") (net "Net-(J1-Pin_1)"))
 (segment (start 141.35 66.5) (end 127.5 66.5) (width 0.2) (layer "F.Cu") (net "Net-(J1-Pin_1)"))
 (segment (start 117.4875 86.711) (end 117.4875 62.3935) (width 0.2) (layer "B.Cu") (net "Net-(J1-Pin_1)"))
 (segment (start 117.4875 62.3935) (end 122.056 57.825) (width 0.2) (layer "B.Cu") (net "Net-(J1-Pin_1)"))
 (segment (start 130.5 54) (end 146.5 54) (width 0.2) (layer "F.Cu") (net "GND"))
 (segment (start 146.5 54) (end 147 54.5) (width 0.2) (layer "F.Cu") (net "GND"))
 (segment (start 129.676 57.825) (end 129.676 55.176) (width 0.2) (layer "F.Cu") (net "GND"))
 (segment (start 147 54.5) (end 147 59) (width 0.2) (layer "F.Cu") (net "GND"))
 (segment (start 145.665 60.335) (end 142.435 60.335) (width 0.2) (layer "F.Cu") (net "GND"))
 (segment (start 129.676 55.176) (end 128.5 54) (width 0.2) (layer "F.Cu") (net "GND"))
 (segment (start 129.676 54.824) (end 130.5 54) (width 0.2) (layer "F.Cu") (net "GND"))
 (segment (start 147 59) (end 145.665 60.335) (width 0.2) (layer "F.Cu") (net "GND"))
 (segment (start 128.5 54) (end 96.5 54) (width 0.2) (layer "F.Cu") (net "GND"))
 (segment (start 129.676 55.176) (end 129.676 54.824) (width 0.2) (layer "F.Cu") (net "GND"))
 (segment (start 145.56 94.94) (end 138.9 94.94) (width 0.2) (layer "B.Cu") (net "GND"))
 (segment (start 146.165 60.335) (end 142.435 60.335) (width 0.2) (layer "B.Cu") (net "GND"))
 (segment (start 146.335 60.335) (end 147 61) (width 0.2) (layer "B.Cu") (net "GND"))
 (segment (start 147 93.5) (end 145.56 94.94) (width 0.2) (layer "B.Cu") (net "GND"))
 (segment (start 147 61) (end 147 93.5) (width 0.2) (layer "B.Cu") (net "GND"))
 (segment (start 142.435 60.335) (end 146.335 60.335) (width 0.2) (layer "B.Cu") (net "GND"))
 (segment (start 128.5 90) (end 138.76 90) (width 0.2) (layer "F.Cu") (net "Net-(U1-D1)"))
 (segment (start 127.6475 89.1475) (end 128.5 90) (width 0.2) (layer "F.Cu") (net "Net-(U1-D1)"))
 (segment (start 138.76 90) (end 138.9 89.86) (width 0.2) (layer "F.Cu") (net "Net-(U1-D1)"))
 (segment (start 127.6475 86.711) (end 127.6475 89.1475) (width 0.2) (layer "F.Cu") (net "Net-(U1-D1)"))
 (segment (start 142.5 89) (end 141.64 89.86) (width 0.2) (layer "B.Cu") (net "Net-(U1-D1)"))
 (segment (start 142.5 78.5) (end 142.5 89) (width 0.2) (layer "B.Cu") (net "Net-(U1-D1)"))
 (segment (start 141.64 89.86) (end 138.9 89.86) (width 0.2) (layer "B.Cu") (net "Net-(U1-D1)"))
 (segment (start 140.31 76.31) (end 142.5 78.5) (width 0.2) (layer "B.Cu") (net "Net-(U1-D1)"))
 (segment (start 137.5 76.31) (end 140.31 76.31) (width 0.2) (layer "B.Cu") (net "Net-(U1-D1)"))
 (segment (start 124 83) (end 118.5 83) (width 0.2) (layer "F.Cu") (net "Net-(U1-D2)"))
 (segment (start 106.585 61.085) (end 106.585 57.965) (width 0.2) (layer "F.Cu") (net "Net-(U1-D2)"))
 (segment (start 118.5 62.5) (end 117.5 61.5) (width 0.2) (layer "F.Cu") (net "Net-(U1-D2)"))
 (segment (start 117.5 61.5) (end 107 61.5) (width 0.2) (layer "F.Cu") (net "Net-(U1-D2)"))
 (segment (start 125.1075 86.711) (end 125.1075 84.1075) (width 0.2) (layer "F.Cu") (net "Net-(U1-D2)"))
 (segment (start 118.5 83) (end 118.5 62.5) (width 0.2) (layer "F.Cu") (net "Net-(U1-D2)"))
 (segment (start 125.1075 84.1075) (end 124 83) (width 0.2) (layer "F.Cu") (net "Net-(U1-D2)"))
 (segment (start 107 61.5) (end 106.585 61.085) (width 0.2) (layer "F.Cu") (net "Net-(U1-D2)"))
 (segment (start 122.5675 86.711) (end 122.5675 84.0675) (width 0.2) (layer "F.Cu") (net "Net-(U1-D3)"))
 (segment (start 107.14 72.5) (end 106.585 73.055) (width 0.2) (layer "F.Cu") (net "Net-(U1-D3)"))
 (segment (start 122.5675 84.0675) (end 122.124 83.624) (width 0.2) (layer "F.Cu") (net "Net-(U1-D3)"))
 (segment (start 112.124 83.624) (end 111.5 83) (width 0.2) (layer "F.Cu") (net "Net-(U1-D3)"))
 (segment (start 111.5 72.5) (end 107.14 72.5) (width 0.2) (layer "F.Cu") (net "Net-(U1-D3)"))
 (segment (start 111.5 83) (end 111.5 72.5) (width 0.2) (layer "F.Cu") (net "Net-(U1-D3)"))
 (segment (start 122.124 83.624) (end 112.124 83.624) (width 0.2) (layer "F.Cu") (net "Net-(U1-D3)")))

